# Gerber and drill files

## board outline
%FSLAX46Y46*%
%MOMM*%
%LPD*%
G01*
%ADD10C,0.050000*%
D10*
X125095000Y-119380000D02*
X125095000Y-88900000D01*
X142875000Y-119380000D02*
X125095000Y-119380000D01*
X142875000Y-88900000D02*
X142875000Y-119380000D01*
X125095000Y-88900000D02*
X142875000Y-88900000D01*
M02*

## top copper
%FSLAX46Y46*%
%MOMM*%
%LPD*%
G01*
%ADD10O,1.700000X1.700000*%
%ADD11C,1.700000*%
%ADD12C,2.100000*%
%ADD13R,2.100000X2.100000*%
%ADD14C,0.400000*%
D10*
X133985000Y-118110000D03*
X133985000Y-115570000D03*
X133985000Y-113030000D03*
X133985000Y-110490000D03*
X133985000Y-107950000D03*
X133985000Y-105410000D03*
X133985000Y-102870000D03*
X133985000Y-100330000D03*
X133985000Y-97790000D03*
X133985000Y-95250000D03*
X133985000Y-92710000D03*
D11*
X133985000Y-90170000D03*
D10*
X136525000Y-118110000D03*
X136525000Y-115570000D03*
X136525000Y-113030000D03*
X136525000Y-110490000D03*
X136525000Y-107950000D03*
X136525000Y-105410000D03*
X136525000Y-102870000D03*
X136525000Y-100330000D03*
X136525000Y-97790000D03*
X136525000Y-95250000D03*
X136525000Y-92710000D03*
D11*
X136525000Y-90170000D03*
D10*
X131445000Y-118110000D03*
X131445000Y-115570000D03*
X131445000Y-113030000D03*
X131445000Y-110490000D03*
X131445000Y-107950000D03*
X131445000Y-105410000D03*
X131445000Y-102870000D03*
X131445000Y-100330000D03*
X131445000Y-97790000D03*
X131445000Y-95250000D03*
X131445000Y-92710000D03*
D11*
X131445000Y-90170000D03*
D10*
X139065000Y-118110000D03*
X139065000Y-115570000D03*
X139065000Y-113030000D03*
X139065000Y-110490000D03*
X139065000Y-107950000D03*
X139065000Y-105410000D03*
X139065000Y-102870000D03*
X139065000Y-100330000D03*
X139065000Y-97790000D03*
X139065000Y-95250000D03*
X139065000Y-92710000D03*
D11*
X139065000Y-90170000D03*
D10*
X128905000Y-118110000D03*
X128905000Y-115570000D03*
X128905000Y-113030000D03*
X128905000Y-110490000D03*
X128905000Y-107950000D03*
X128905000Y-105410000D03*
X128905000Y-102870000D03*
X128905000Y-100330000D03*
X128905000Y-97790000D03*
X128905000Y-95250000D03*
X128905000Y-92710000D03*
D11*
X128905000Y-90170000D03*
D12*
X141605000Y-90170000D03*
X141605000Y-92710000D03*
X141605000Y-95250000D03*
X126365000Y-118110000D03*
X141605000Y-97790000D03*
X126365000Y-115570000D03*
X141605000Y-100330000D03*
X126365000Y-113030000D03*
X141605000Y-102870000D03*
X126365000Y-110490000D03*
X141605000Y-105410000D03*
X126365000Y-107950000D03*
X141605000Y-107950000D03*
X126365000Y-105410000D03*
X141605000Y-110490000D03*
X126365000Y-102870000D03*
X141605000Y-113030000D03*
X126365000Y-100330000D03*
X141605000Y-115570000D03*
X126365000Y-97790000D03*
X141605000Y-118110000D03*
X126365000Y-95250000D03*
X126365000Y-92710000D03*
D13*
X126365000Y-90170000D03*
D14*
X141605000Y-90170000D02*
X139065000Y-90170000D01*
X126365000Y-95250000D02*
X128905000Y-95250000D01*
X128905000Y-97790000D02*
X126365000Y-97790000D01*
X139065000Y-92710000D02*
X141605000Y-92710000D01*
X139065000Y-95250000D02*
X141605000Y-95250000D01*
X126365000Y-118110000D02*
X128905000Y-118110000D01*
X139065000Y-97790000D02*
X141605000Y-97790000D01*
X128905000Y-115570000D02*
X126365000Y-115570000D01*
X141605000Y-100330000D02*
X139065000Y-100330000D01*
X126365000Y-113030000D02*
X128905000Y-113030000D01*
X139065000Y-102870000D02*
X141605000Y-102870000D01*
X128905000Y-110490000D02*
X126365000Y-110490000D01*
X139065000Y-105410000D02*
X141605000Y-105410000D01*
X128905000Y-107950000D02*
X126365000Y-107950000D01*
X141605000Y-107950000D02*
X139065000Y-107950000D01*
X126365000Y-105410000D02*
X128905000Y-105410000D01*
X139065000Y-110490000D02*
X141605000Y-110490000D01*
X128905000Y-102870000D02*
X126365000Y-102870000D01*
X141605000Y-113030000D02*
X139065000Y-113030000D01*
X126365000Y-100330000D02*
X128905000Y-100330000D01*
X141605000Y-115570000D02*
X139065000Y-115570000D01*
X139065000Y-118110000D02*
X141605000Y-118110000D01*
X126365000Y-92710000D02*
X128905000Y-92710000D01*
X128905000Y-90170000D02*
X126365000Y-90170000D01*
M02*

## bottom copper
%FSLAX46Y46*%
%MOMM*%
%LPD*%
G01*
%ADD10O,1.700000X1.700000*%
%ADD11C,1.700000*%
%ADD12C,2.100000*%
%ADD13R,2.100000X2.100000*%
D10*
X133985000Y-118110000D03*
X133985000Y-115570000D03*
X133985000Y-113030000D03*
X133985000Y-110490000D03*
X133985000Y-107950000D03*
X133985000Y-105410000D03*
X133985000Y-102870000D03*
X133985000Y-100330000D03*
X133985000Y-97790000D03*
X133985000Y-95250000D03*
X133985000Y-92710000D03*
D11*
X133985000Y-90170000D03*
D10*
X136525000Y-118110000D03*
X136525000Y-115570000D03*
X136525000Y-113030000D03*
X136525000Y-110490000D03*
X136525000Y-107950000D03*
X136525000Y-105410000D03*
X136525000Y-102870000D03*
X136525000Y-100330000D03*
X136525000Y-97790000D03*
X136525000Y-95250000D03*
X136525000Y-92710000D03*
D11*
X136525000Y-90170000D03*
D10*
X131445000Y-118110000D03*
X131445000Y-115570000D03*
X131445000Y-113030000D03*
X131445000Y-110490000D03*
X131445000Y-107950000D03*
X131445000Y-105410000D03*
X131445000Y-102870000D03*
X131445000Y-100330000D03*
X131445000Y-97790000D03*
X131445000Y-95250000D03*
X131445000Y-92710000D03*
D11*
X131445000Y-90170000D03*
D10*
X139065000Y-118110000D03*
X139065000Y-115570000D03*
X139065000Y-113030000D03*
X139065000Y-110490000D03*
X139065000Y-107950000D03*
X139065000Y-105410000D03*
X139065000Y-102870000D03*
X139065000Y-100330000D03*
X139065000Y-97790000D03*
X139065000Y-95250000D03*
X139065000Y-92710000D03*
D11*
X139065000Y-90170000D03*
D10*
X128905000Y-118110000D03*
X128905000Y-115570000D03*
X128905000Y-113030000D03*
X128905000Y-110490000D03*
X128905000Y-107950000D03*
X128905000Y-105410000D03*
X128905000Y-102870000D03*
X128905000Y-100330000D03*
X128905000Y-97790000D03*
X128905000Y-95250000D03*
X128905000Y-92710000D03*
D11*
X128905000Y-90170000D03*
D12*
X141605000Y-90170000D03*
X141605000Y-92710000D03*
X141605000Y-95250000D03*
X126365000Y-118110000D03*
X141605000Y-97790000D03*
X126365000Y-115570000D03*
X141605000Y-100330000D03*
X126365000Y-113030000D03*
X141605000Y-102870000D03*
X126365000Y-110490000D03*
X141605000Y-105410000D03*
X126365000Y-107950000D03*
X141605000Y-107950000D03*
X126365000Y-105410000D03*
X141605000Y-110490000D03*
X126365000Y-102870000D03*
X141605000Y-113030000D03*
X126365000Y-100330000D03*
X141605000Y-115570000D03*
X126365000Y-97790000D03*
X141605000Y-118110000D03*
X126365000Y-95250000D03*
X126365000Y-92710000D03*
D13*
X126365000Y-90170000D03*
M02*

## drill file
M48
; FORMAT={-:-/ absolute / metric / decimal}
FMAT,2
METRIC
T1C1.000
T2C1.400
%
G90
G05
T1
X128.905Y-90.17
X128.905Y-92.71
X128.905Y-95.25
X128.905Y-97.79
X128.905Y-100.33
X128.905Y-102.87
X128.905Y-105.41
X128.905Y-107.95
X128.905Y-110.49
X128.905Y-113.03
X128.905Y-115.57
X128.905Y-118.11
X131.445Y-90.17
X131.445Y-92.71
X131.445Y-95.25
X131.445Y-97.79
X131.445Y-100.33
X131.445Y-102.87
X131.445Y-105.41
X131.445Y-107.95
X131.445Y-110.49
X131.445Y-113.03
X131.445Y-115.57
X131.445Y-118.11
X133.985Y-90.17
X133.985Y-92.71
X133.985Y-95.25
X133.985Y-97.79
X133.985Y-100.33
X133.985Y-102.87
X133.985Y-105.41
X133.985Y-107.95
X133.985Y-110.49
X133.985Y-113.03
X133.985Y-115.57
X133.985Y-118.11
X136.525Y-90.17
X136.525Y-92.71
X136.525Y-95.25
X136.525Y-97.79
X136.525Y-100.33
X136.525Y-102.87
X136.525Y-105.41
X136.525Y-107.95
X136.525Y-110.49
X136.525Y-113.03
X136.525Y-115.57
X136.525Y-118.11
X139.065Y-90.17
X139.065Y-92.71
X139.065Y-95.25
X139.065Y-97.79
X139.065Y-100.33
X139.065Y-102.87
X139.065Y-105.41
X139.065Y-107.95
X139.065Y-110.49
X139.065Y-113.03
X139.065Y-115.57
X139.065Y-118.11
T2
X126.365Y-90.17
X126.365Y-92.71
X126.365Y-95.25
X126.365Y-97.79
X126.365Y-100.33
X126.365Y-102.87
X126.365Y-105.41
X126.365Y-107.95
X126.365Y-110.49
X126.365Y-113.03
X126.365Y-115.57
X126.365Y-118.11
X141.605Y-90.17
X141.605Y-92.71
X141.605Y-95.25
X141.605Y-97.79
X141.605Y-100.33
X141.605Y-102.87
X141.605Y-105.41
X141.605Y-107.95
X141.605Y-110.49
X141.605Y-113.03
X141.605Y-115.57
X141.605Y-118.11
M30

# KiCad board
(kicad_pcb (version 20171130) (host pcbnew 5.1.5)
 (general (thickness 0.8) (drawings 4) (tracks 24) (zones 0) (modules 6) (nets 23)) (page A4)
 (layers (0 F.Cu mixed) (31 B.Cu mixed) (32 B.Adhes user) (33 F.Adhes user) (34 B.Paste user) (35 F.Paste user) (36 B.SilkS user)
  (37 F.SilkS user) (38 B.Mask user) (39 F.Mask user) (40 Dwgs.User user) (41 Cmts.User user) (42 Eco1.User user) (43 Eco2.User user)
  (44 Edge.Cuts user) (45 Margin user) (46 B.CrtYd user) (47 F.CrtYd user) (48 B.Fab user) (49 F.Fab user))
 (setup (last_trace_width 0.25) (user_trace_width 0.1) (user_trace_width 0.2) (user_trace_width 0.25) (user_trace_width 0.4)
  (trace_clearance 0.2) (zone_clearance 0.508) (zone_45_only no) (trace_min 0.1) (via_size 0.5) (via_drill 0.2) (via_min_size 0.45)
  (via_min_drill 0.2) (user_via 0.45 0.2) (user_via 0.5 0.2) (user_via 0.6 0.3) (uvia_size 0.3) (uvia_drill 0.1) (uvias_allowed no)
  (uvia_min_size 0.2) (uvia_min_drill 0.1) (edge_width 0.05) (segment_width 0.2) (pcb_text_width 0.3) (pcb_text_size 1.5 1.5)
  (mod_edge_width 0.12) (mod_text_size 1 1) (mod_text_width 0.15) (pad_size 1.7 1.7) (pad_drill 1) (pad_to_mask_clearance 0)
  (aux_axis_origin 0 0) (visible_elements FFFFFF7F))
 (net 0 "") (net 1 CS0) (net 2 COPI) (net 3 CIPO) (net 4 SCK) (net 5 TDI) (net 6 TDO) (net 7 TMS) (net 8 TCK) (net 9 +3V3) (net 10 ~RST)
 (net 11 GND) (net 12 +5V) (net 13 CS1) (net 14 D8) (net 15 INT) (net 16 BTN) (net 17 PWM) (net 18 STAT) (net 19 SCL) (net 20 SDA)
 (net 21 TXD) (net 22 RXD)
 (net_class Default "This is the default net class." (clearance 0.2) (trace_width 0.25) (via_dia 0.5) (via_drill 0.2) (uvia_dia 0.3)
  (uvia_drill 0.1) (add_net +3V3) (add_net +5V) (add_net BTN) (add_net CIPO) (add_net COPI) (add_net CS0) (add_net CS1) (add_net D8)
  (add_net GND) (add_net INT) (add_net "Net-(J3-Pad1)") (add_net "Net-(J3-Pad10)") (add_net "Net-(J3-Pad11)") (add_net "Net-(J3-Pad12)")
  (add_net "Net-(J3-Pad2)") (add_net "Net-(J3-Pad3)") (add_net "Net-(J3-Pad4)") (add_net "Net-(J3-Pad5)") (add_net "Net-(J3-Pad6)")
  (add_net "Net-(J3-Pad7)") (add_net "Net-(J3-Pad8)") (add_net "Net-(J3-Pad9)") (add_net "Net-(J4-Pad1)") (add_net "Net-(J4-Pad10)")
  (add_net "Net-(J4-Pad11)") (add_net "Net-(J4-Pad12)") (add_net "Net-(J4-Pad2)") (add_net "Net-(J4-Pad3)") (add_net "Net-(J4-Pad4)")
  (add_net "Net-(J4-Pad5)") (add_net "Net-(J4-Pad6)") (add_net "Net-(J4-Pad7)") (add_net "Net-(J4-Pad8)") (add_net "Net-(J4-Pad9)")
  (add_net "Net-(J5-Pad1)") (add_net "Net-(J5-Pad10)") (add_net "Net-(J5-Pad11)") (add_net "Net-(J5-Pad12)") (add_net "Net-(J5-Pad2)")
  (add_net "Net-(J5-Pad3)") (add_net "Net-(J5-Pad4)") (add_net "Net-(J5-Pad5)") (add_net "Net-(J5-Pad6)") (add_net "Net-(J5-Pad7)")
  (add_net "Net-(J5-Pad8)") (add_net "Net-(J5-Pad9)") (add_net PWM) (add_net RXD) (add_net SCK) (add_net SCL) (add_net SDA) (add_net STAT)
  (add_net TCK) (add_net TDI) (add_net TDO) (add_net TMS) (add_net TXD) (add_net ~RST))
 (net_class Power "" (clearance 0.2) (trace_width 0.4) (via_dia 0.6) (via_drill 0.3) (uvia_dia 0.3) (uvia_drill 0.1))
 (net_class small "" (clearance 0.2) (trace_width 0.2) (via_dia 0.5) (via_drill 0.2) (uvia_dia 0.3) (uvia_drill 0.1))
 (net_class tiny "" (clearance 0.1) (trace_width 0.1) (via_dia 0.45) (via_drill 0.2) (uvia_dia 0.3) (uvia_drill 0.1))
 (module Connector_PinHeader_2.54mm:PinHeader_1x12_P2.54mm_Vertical (layer F.Cu) (at 133.985 90.17)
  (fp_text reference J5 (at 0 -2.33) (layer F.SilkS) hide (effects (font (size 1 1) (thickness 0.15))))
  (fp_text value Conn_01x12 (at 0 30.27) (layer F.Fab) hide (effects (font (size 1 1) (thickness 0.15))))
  (pad 12 thru_hole oval (at 0 27.94) (size 1.7 1.7) (drill 1) (layers *.Cu *.Mask))
  (pad 11 thru_hole oval (at 0 25.4) (size 1.7 1.7) (drill 1) (layers *.Cu *.Mask))
  (pad 10 thru_hole oval (at 0 22.86) (size 1.7 1.7) (drill 1) (layers *.Cu *.Mask))
  (pad 9 thru_hole oval (at 0 20.32) (size 1.7 1.7) (drill 1) (layers *.Cu *.Mask))
  (pad 8 thru_hole oval (at 0 17.78) (size 1.7 1.7) (drill 1) (layers *.Cu *.Mask))
  (pad 7 thru_hole oval (at 0 15.24) (size 1.7 1.7) (drill 1) (layers *.Cu *.Mask))
  (pad 6 thru_hole oval (at 0 12.7) (size 1.7 1.7) (drill 1) (layers *.Cu *.Mask))
  (pad 5 thru_hole oval (at 0 10.16) (size 1.7 1.7) (drill 1) (layers *.Cu *.Mask))
  (pad 4 thru_hole oval (at 0 7.62) (size 1.7 1.7) (drill 1) (layers *.Cu *.Mask))
  (pad 3 thru_hole oval (at 0 5.08) (size 1.7 1.7) (drill 1) (layers *.Cu *.Mask))
  (pad 2 thru_hole oval (at 0 2.54) (size 1.7 1.7) (drill 1) (layers *.Cu *.Mask))
  (pad 1 thru_hole circle (at 0 0) (size 1.7 1.7) (drill 1) (layers *.Cu *.Mask)))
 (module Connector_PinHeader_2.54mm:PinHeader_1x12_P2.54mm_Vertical (layer F.Cu) (at 136.525 90.17)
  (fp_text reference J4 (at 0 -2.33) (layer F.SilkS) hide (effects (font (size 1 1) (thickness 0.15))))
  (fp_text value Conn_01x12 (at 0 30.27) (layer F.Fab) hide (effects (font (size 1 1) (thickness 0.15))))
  (pad 12 thru_hole oval (at 0 27.94) (size 1.7 1.7) (drill 1) (layers *.Cu *.Mask))
  (pad 11 thru_hole oval (at 0 25.4) (size 1.7 1.7) (drill 1) (layers *.Cu *.Mask))
  (pad 10 thru_hole oval (at 0 22.86) (size 1.7 1.7) (drill 1) (layers *.Cu *.Mask))
  (pad 9 thru_hole oval (at 0 20.32) (size 1.7 1.7) (drill 1) (layers *.Cu *.Mask))
  (pad 8 thru_hole oval (at 0 17.78) (size 1.7 1.7) (drill 1) (layers *.Cu *.Mask))
  (pad 7 thru_hole oval (at 0 15.24) (size 1.7 1.7) (drill 1) (layers *.Cu *.Mask))
  (pad 6 thru_hole oval (at 0 12.7) (size 1.7 1.7) (drill 1) (layers *.Cu *.Mask))
  (pad 5 thru_hole oval (at 0 10.16) (size 1.7 1.7) (drill 1) (layers *.Cu *.Mask))
  (pad 4 thru_hole oval (at 0 7.62) (size 1.7 1.7) (drill 1) (layers *.Cu *.Mask))
  (pad 3 thru_hole oval (at 0 5.08) (size 1.7 1.7) (drill 1) (layers *.Cu *.Mask))
  (pad 2 thru_hole oval (at 0 2.54) (size 1.7 1.7) (drill 1) (layers *.Cu *.Mask))
  (pad 1 thru_hole circle (at 0 0) (size 1.7 1.7) (drill 1) (layers *.Cu *.Mask)))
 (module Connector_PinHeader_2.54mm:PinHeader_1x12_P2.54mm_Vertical (layer F.Cu) (at 131.445 90.17)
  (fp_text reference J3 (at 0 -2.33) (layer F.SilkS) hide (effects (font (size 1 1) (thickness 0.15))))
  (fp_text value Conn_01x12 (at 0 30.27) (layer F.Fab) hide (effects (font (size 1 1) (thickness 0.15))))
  (pad 12 thru_hole oval (at 0 27.94) (size 1.7 1.7) (drill 1) (layers *.Cu *.Mask))
  (pad 11 thru_hole oval (at 0 25.4) (size 1.7 1.7) (drill 1) (layers *.Cu *.Mask))
  (pad 10 thru_hole oval (at 0 22.86) (size 1.7 1.7) (drill 1) (layers *.Cu *.Mask))
  (pad 9 thru_hole oval (at 0 20.32) (size 1.7 1.7) (drill 1) (layers *.Cu *.Mask))
  (pad 8 thru_hole oval (at 0 17.78) (size 1.7 1.7) (drill 1) (layers *.Cu *.Mask))
  (pad 7 thru_hole oval (at 0 15.24) (size 1.7 1.7) (drill 1) (layers *.Cu *.Mask))
  (pad 6 thru_hole oval (at 0 12.7) (size 1.7 1.7) (drill 1) (layers *.Cu *.Mask))
  (pad 5 thru_hole oval (at 0 10.16) (size 1.7 1.7) (drill 1) (layers *.Cu *.Mask))
  (pad 4 thru_hole oval (at 0 7.62) (size 1.7 1.7) (drill 1) (layers *.Cu *.Mask))
  (pad 3 thru_hole oval (at 0 5.08) (size 1.7 1.7) (drill 1) (layers *.Cu *.Mask))
  (pad 2 thru_hole oval (at 0 2.54) (size 1.7 1.7) (drill 1) (layers *.Cu *.Mask))
  (pad 1 thru_hole circle (at 0 0) (size 1.7 1.7) (drill 1) (layers *.Cu *.Mask)))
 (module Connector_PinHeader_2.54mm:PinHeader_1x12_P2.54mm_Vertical (layer F.Cu) (at 139.065 90.17)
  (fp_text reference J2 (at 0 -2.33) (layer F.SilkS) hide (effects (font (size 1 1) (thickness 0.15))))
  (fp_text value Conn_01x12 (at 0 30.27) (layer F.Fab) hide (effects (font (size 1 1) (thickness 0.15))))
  (pad 12 thru_hole oval (at 0 27.94) (size 1.7 1.7) (drill 1) (layers *.Cu *.Mask) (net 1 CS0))
  (pad 11 thru_hole oval (at 0 25.4) (size 1.7 1.7) (drill 1) (layers *.Cu *.Mask) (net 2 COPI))
  (pad 10 thru_hole oval (at 0 22.86) (size 1.7 1.7) (drill 1) (layers *.Cu *.Mask) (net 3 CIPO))
  (pad 9 thru_hole oval (at 0 20.32) (size 1.7 1.7) (drill 1) (layers *.Cu *.Mask) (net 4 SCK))
  (pad 8 thru_hole oval (at 0 17.78) (size 1.7 1.7) (drill 1) (layers *.Cu *.Mask) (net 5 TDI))
  (pad 7 thru_hole oval (at 0 15.24) (size 1.7 1.7) (drill 1) (layers *.Cu *.Mask) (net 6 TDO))
  (pad 6 thru_hole oval (at 0 12.7) (size 1.7 1.7) (drill 1) (layers *.Cu *.Mask) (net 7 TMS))
  (pad 5 thru_hole oval (at 0 10.16) (size 1.7 1.7) (drill 1) (layers *.Cu *.Mask) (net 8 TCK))
  (pad 4 thru_hole oval (at 0 7.62) (size 1.7 1.7) (drill 1) (layers *.Cu *.Mask) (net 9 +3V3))
  (pad 3 thru_hole oval (at 0 5.08) (size 1.7 1.7) (drill 1) (layers *.Cu *.Mask) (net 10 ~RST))
  (pad 2 thru_hole oval (at 0 2.54) (size 1.7 1.7) (drill 1) (layers *.Cu *.Mask) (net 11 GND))
  (pad 1 thru_hole circle (at 0 0) (size 1.7 1.7) (drill 1) (layers *.Cu *.Mask) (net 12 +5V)))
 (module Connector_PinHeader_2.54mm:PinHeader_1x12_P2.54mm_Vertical (layer F.Cu) (at 128.905 90.17)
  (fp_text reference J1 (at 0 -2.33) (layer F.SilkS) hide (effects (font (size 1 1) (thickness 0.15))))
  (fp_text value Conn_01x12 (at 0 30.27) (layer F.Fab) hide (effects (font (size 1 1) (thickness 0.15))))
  (pad 12 thru_hole oval (at 0 27.94) (size 1.7 1.7) (drill 1) (layers *.Cu *.Mask) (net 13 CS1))
  (pad 11 thru_hole oval (at 0 25.4) (size 1.7 1.7) (drill 1) (layers *.Cu *.Mask) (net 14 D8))
  (pad 10 thru_hole oval (at 0 22.86) (size 1.7 1.7) (drill 1) (layers *.Cu *.Mask) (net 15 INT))
  (pad 9 thru_hole oval (at 0 20.32) (size 1.7 1.7) (drill 1) (layers *.Cu *.Mask) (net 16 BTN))
  (pad 8 thru_hole oval (at 0 17.78) (size 1.7 1.7) (drill 1) (layers *.Cu *.Mask) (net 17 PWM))
  (pad 7 thru_hole oval (at 0 15.24) (size 1.7 1.7) (drill 1) (layers *.Cu *.Mask) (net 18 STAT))
  (pad 6 thru_hole oval (at 0 12.7) (size 1.7 1.7) (drill 1) (layers *.Cu *.Mask) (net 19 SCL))
  (pad 5 thru_hole oval (at 0 10.16) (size 1.7 1.7) (drill 1) (layers *.Cu *.Mask) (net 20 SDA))
  (pad 4 thru_hole oval (at 0 7.62) (size 1.7 1.7) (drill 1) (layers *.Cu *.Mask) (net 11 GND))
  (pad 3 thru_hole oval (at 0 5.08) (size 1.7 1.7) (drill 1) (layers *.Cu *.Mask) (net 11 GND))
  (pad 2 thru_hole oval (at 0 2.54) (size 1.7 1.7) (drill 1) (layers *.Cu *.Mask) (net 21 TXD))
  (pad 1 thru_hole circle (at 0 0) (size 1.7 1.7) (drill 1) (layers *.Cu *.Mask) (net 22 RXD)))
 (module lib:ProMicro (layer F.Cu) (at 126.365 90.17)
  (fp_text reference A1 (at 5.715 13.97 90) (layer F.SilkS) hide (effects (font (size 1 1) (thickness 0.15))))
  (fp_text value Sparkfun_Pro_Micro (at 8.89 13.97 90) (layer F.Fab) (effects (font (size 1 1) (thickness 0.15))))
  (pad 24 thru_hole circle (at 15.24 0) (size 2.1 2.1) (drill 1.4) (layers *.Cu *.Mask) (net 12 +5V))
  (pad 23 thru_hole circle (at 15.24 2.54) (size 2.1 2.1) (drill 1.4) (layers *.Cu *.Mask) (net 11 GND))
  (pad 22 thru_hole circle (at 15.24 5.08) (size 2.1 2.1) (drill 1.4) (layers *.Cu *.Mask) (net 10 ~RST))
  (pad 12 thru_hole circle (at 0 27.94) (size 2.1 2.1) (drill 1.4) (layers *.Cu *.Mask) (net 13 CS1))
  (pad 21 thru_hole circle (at 15.24 7.62) (size 2.1 2.1) (drill 1.4) (layers *.Cu *.Mask) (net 9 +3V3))
  (pad 11 thru_hole circle (at 0 25.4) (size 2.1 2.1) (drill 1.4) (layers *.Cu *.Mask) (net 14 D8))
  (pad 20 thru_hole circle (at 15.24 10.16) (size 2.1 2.1) (drill 1.4) (layers *.Cu *.Mask) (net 8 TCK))
  (pad 10 thru_hole circle (at 0 22.86) (size 2.1 2.1) (drill 1.4) (layers *.Cu *.Mask) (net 15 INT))
  (pad 19 thru_hole circle (at 15.24 12.7) (size 2.1 2.1) (drill 1.4) (layers *.Cu *.Mask) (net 7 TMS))
  (pad 9 thru_hole circle (at 0 20.32) (size 2.1 2.1) (drill 1.4) (layers *.Cu *.Mask) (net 16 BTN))
  (pad 18 thru_hole circle (at 15.24 15.24) (size 2.1 2.1) (drill 1.4) (layers *.Cu *.Mask) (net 6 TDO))
  (pad 8 thru_hole circle (at 0 17.78) (size 2.1 2.1) (drill 1.4) (layers *.Cu *.Mask) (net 17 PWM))
  (pad 17 thru_hole circle (at 15.24 17.78) (size 2.1 2.1) (drill 1.4) (layers *.Cu *.Mask) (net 5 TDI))
  (pad 7 thru_hole circle (at 0 15.24) (size 2.1 2.1) (drill 1.4) (layers *.Cu *.Mask) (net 18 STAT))
  (pad 16 thru_hole circle (at 15.24 20.32) (size 2.1 2.1) (drill 1.4) (layers *.Cu *.Mask) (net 4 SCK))
  (pad 6 thru_hole circle (at 0 12.7) (size 2.1 2.1) (drill 1.4) (layers *.Cu *.Mask) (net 19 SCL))
  (pad 15 thru_hole circle (at 15.24 22.86) (size 2.1 2.1) (drill 1.4) (layers *.Cu *.Mask) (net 3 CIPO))
  (pad 5 thru_hole circle (at 0 10.16) (size 2.1 2.1) (drill 1.4) (layers *.Cu *.Mask) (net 20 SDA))
  (pad 14 thru_hole circle (at 15.24 25.4) (size 2.1 2.1) (drill 1.4) (layers *.Cu *.Mask) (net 2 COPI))
  (pad 4 thru_hole circle (at 0 7.62) (size 2.1 2.1) (drill 1.4) (layers *.Cu *.Mask) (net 11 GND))
  (pad 13 thru_hole circle (at 15.24 27.94) (size 2.1 2.1) (drill 1.4) (layers *.Cu *.Mask) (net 1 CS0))
  (pad 3 thru_hole circle (at 0 5.08) (size 2.1 2.1) (drill 1.4) (layers *.Cu *.Mask) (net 11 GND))
  (pad 2 thru_hole circle (at 0 2.54) (size 2.1 2.1) (drill 1.4) (layers *.Cu *.Mask) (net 21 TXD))
  (pad 1 thru_hole rect (at 0 0) (size 2.1 2.1) (drill 1.4) (layers *.Cu *.Mask) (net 22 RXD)))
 (gr_line (start 125.095 119.38) (end 125.095 88.9) (layer Edge.Cuts) (width 0.05))
 (gr_line (start 142.875 119.38) (end 125.095 119.38) (layer Edge.Cuts) (width 0.05))
 (gr_line (start 142.875 88.9) (end 142.875 119.38) (layer Edge.Cuts) (width 0.05))
 (gr_line (start 125.095 88.9) (end 142.875 88.9) (layer Edge.Cuts) (width 0.05))
 (segment (start 141.605 90.17) (end 139.065 90.17) (width 0.4) (layer F.Cu) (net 12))
 (segment (start 126.365 95.25) (end 128.905 95.25) (width 0.4) (layer F.Cu) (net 11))
 (segment (start 128.905 97.79) (end 126.365 97.79) (width 0.4) (layer F.Cu) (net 11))
 (segment (start 139.065 92.71) (end 141.605 92.71) (width 0.4) (layer F.Cu) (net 11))
 (segment (start 139.065 95.25) (end 141.605 95.25) (width 0.4) (layer F.Cu) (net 10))
 (segment (start 126.365 118.11) (end 128.905 118.11) (width 0.4) (layer F.Cu) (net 13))
 (segment (start 139.065 97.79) (end 141.605 97.79) (width 0.4) (layer F.Cu) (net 9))
 (segment (start 128.905 115.57) (end 126.365 115.57) (width 0.4) (layer F.Cu) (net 14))
 (segment (start 141.605 100.33) (end 139.065 100.33) (width 0.4) (layer F.Cu) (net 8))
 (segment (start 126.365 113.03) (end 128.905 113.03) (width 0.4) (layer F.Cu) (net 15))
 (segment (start 139.065 102.87) (end 141.605 102.87) (width 0.4) (layer F.Cu) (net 7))
 (segment (start 128.905 110.49) (end 126.365 110.49) (width 0.4) (layer F.Cu) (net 16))
 (segment (start 139.065 105.41) (end 141.605 105.41) (width 0.4) (layer F.Cu) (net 6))
 (segment (start 128.905 107.95) (end 126.365 107.95) (width 0.4) (layer F.Cu) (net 17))
 (segment (start 141.605 107.95) (end 139.065 107.95) (width 0.4) (layer F.Cu) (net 5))
 (segment (start 126.365 105.41) (end 128.905 105.41) (width 0.4) (layer F.Cu) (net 18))
 (segment (start 139.065 110.49) (end 141.605 110.49) (width 0.4) (layer F.Cu) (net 4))
 (segment (start 128.905 102.87) (end 126.365 102.87) (width 0.4) (layer F.Cu) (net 19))
 (segment (start 141.605 113.03) (end 139.065 113.03) (width 0.4) (layer F.Cu) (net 3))
 (segment (start 126.365 100.33) (end 128.905 100.33) (width 0.4) (layer F.Cu) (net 20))
 (segment (start 141.605 115.57) (end 139.065 115.57) (width 0.4) (layer F.Cu) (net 2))
 (segment (start 139.065 118.11) (end 141.605 118.11) (width 0.4) (layer F.Cu) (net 1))
 (segment (start 126.365 92.71) (end 128.905 92.71) (width 0.4) (layer F.Cu) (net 21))
 (segment (start 128.905 90.17) (end 126.365 90.17) (width 0.4) (layer F.Cu) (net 22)))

